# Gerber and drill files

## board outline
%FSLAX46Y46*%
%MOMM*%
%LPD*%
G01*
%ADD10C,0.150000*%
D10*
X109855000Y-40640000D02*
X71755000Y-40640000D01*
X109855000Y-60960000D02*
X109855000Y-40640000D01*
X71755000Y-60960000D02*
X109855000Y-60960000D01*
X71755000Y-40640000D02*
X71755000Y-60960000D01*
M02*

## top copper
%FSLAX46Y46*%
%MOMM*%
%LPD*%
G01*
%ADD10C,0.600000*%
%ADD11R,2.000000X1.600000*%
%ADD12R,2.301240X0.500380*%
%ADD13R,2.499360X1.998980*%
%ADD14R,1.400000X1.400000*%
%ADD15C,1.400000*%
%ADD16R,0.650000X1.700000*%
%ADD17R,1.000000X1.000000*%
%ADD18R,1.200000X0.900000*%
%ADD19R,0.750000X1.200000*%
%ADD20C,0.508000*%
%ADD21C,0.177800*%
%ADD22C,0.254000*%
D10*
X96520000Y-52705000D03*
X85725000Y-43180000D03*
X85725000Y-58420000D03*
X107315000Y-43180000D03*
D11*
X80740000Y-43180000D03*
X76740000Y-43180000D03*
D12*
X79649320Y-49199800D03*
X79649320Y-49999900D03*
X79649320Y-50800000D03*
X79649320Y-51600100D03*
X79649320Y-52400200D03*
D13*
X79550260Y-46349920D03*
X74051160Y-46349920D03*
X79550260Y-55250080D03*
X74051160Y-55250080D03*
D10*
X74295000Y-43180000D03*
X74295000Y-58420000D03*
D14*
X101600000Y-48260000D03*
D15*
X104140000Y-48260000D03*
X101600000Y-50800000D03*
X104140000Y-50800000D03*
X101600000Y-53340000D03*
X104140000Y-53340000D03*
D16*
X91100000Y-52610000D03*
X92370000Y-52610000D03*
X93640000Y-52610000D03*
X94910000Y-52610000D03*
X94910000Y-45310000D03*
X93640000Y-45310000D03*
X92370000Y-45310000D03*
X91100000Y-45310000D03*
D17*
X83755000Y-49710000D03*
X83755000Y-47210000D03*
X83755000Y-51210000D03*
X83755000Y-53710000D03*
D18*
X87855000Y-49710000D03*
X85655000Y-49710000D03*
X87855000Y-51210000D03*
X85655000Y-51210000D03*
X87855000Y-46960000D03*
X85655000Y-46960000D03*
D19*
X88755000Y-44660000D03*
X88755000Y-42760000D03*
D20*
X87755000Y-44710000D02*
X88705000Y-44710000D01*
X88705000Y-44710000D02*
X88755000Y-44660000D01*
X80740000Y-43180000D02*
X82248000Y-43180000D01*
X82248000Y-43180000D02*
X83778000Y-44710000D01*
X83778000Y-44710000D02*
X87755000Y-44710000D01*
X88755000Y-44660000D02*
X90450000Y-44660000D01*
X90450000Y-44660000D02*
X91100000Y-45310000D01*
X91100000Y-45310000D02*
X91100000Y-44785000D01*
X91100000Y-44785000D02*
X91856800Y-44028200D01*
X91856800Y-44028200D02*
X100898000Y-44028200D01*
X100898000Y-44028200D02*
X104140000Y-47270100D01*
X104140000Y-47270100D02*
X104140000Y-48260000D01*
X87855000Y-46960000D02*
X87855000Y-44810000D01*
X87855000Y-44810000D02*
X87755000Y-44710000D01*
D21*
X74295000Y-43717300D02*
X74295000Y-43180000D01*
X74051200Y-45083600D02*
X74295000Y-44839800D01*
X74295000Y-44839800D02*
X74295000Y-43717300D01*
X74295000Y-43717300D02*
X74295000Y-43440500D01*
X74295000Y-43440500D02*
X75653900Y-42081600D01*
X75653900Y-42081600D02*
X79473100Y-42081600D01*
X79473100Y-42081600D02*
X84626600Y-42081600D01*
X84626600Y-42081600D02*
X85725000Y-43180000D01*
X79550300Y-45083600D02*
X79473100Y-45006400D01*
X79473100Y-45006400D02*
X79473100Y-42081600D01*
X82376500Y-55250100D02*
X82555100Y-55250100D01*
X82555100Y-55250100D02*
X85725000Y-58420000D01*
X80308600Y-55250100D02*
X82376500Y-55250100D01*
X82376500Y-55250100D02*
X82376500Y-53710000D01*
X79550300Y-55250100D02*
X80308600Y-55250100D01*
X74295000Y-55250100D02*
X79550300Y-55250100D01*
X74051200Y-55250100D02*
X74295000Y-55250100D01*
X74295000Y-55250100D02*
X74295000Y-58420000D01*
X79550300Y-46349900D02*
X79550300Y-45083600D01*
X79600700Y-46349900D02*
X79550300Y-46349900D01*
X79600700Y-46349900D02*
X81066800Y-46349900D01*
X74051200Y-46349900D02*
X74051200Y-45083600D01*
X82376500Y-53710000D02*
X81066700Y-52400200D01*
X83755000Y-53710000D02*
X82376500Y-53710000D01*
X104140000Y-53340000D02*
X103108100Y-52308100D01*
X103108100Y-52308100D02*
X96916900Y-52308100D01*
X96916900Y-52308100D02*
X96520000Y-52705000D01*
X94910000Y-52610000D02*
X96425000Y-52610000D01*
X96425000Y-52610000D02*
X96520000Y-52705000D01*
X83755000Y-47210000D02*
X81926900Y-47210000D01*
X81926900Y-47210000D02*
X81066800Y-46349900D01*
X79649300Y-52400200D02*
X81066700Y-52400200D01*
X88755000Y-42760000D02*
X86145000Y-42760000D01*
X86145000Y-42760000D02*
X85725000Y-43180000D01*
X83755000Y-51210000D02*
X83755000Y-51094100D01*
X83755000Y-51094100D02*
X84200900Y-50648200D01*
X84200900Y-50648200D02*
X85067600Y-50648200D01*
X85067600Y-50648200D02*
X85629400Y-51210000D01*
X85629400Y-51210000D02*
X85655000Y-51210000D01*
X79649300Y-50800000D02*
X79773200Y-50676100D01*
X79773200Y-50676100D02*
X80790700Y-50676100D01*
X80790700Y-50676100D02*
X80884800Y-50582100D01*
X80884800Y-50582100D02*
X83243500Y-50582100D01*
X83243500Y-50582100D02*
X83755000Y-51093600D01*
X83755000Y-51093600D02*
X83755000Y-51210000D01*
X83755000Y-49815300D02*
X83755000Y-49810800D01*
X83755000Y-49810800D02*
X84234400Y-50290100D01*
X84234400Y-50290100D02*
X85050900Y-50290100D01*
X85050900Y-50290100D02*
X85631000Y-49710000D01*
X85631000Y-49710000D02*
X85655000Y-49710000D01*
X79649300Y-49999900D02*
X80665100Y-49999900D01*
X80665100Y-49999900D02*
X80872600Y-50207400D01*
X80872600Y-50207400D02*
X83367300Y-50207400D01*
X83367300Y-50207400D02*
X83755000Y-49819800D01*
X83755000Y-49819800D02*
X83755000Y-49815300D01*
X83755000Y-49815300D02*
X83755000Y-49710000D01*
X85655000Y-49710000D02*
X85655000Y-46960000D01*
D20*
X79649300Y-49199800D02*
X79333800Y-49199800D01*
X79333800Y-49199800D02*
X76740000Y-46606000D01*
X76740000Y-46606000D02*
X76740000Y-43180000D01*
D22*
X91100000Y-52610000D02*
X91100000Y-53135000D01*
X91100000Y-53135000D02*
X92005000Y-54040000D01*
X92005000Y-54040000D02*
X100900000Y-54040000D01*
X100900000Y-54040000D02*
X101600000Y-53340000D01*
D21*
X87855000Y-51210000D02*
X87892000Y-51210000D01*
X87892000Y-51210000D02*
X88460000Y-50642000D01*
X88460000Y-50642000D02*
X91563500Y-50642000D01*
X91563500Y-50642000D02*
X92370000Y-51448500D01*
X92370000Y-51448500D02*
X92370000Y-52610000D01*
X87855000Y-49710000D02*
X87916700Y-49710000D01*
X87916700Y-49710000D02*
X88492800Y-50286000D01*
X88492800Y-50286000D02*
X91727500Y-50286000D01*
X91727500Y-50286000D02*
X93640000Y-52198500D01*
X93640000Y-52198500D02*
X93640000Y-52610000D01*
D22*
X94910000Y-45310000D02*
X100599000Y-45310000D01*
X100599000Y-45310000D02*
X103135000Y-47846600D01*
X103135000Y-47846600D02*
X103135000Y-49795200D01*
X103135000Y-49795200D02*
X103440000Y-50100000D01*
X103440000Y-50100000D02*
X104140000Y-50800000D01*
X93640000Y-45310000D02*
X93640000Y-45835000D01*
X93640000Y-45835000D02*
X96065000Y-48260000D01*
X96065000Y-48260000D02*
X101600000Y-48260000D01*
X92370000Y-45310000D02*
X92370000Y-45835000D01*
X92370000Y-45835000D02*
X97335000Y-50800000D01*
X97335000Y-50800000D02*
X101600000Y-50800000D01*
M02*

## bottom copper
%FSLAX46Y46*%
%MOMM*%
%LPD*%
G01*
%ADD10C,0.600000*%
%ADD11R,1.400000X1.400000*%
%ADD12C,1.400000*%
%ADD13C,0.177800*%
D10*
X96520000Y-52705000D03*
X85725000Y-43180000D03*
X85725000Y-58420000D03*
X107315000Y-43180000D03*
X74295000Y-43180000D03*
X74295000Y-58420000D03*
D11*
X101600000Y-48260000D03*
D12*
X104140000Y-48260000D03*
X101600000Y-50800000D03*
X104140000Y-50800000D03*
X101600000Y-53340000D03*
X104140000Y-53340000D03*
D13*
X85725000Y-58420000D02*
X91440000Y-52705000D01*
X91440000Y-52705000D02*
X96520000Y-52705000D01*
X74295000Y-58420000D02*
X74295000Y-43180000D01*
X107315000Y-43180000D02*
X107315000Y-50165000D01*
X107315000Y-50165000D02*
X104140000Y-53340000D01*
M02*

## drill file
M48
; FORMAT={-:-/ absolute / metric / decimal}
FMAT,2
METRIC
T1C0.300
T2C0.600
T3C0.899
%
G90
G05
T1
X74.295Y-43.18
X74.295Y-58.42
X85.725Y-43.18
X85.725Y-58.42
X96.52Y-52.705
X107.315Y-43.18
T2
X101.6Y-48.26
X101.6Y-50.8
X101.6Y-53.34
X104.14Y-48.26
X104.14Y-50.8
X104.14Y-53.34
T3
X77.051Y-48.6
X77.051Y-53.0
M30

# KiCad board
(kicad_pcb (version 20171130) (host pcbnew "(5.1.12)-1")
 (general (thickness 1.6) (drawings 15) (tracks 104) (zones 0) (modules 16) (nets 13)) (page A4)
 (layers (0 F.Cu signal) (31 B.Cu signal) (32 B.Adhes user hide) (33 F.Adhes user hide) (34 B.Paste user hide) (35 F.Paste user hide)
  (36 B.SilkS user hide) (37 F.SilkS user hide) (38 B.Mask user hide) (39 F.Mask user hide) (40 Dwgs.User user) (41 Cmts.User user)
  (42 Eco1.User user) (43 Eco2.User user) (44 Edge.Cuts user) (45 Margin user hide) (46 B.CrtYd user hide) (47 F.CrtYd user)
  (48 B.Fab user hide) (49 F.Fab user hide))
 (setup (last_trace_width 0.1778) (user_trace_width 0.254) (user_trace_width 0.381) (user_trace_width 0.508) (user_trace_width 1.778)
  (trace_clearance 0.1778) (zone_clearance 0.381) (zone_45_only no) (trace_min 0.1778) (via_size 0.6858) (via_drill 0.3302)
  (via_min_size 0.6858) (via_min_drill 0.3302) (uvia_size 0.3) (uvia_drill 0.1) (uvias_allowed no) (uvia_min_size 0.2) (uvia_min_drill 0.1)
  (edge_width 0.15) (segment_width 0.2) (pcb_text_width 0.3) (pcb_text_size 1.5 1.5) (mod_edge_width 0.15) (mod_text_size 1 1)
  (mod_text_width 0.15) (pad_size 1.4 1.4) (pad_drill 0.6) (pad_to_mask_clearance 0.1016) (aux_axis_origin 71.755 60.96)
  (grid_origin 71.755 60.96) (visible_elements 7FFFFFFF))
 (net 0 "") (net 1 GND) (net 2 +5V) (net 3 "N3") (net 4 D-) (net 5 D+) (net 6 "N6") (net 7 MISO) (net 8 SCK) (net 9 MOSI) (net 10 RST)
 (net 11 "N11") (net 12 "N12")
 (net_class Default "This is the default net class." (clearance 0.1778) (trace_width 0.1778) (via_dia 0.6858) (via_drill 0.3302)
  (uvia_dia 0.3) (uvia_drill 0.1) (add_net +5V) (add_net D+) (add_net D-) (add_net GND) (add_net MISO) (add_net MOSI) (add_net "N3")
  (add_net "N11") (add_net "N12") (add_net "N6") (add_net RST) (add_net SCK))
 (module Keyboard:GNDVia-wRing (layer F.Cu) (at 96.52 52.705)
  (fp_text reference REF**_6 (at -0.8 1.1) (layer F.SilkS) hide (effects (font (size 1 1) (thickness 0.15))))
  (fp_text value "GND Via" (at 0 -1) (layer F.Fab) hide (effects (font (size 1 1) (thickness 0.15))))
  (pad GND thru_hole circle (at 0 0) (size 0.6 0.6) (drill 0.3) (layers *.Cu) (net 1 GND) (zone_connect 2)))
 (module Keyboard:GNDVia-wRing (layer F.Cu) (at 85.725 43.18)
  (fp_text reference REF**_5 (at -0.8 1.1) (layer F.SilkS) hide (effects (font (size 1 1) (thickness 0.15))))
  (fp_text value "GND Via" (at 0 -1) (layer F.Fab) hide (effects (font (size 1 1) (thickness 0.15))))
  (pad GND thru_hole circle (at 0 0) (size 0.6 0.6) (drill 0.3) (layers *.Cu) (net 1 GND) (zone_connect 2)))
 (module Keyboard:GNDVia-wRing (layer F.Cu) (at 85.725 58.42)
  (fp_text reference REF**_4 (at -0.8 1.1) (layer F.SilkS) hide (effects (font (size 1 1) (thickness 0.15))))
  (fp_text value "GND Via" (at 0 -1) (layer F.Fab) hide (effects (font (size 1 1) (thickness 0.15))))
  (pad GND thru_hole circle (at 0 0) (size 0.6 0.6) (drill 0.3) (layers *.Cu) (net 1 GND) (zone_connect 2)))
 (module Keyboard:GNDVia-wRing (layer F.Cu) (at 107.315 43.18)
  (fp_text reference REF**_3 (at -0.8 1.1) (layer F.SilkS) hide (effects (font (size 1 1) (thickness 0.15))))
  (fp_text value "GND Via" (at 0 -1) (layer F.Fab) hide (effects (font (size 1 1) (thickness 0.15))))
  (pad GND thru_hole circle (at 0 0) (size 0.6 0.6) (drill 0.3) (layers *.Cu) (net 1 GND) (zone_connect 2)))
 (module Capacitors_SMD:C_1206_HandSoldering (layer F.Cu) (at 78.74 43.18 180)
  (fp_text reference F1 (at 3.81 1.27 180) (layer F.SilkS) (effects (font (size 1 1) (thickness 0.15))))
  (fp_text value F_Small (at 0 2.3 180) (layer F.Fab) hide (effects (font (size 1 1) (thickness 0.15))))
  (pad 1 smd rect (at -2 0 180) (size 2 1.6) (layers F.Cu F.Paste F.Mask) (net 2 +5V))
  (pad 2 smd rect (at 2 0 180) (size 2 1.6) (layers F.Cu F.Paste F.Mask) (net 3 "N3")))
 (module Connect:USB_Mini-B (layer F.Cu) (at 76.2 50.8)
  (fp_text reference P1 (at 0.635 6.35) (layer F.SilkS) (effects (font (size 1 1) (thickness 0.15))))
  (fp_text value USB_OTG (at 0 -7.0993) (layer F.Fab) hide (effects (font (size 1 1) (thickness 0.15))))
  (pad 1 smd rect (at 3.44932 -1.6002) (size 2.30124 0.50038) (layers F.Cu F.Paste F.Mask) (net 3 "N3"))
  (pad 2 smd rect (at 3.44932 -0.8001) (size 2.30124 0.50038) (layers F.Cu F.Paste F.Mask) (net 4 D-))
  (pad 3 smd rect (at 3.44932 0) (size 2.30124 0.50038) (layers F.Cu F.Paste F.Mask) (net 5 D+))
  (pad 4 smd rect (at 3.44932 0.8001) (size 2.30124 0.50038) (layers F.Cu F.Paste F.Mask) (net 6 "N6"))
  (pad 5 smd rect (at 3.44932 1.6002) (size 2.30124 0.50038) (layers F.Cu F.Paste F.Mask) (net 1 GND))
  (pad 6 smd rect (at 3.35026 -4.45008) (size 2.49936 1.99898) (layers F.Cu F.Paste F.Mask) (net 1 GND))
  (pad 6 smd rect (at -2.14884 -4.45008) (size 2.49936 1.99898) (layers F.Cu F.Paste F.Mask) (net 1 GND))
  (pad 6 smd rect (at 3.35026 4.45008) (size 2.49936 1.99898) (layers F.Cu F.Paste F.Mask) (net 1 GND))
  (pad 6 smd rect (at -2.14884 4.45008) (size 2.49936 1.99898) (layers F.Cu F.Paste F.Mask) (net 1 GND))
  (pad "" np_thru_hole circle (at 0.8509 -2.19964) (size 0.89916 0.89916) (drill 0.89916) (layers *.Cu *.Mask F.SilkS))
  (pad "" np_thru_hole circle (at 0.8509 2.19964) (size 0.89916 0.89916) (drill 0.89916) (layers *.Cu *.Mask F.SilkS)))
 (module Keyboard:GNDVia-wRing (layer F.Cu) (at 74.295 43.18)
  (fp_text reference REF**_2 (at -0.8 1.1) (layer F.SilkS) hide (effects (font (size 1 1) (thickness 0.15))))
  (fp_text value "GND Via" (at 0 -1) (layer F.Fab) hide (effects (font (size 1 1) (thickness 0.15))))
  (pad GND thru_hole circle (at 0 0) (size 0.6 0.6) (drill 0.3) (layers *.Cu) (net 1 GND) (zone_connect 2)))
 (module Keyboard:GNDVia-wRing (layer F.Cu) (at 74.295 58.42)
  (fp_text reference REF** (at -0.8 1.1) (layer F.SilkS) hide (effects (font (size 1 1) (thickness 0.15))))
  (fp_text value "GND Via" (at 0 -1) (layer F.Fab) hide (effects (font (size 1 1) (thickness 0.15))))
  (pad GND thru_hole circle (at 0 0) (size 0.6 0.6) (drill 0.3) (layers *.Cu) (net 1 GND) (zone_connect 2)))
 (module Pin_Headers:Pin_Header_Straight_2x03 (layer F.Cu) (at 101.6 48.26)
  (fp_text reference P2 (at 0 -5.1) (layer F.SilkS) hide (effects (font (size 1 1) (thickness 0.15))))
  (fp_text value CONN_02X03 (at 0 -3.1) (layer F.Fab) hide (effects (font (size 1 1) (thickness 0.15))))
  (pad 1 thru_hole rect (at 0 0) (size 1.4 1.4) (drill 0.6) (layers *.Cu *.Mask F.SilkS) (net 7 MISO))
  (pad 2 thru_hole circle (at 2.54 0) (size 1.4 1.4) (drill 0.6) (layers *.Cu *.Mask F.SilkS) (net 2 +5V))
  (pad 3 thru_hole circle (at 0 2.54) (size 1.4 1.4) (drill 0.6) (layers *.Cu *.Mask F.SilkS) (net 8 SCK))
  (pad 4 thru_hole circle (at 2.54 2.54) (size 1.4 1.4) (drill 0.6) (layers *.Cu *.Mask F.SilkS) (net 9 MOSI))
  (pad 5 thru_hole circle (at 0 5.08) (size 1.4 1.4) (drill 0.6) (layers *.Cu *.Mask F.SilkS) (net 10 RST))
  (pad 6 thru_hole circle (at 2.54 5.08) (size 1.4 1.4) (drill 0.6) (layers *.Cu *.Mask F.SilkS) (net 1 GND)))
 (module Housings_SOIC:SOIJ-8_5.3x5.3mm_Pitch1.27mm (layer F.Cu) (at 93.005 48.96 90)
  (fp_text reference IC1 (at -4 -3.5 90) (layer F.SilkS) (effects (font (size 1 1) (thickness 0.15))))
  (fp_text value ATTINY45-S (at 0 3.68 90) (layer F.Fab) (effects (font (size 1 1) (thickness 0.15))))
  (pad 1 smd rect (at -3.65 -1.905 90) (size 1.7 0.65) (layers F.Cu F.Paste F.Mask) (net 10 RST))
  (pad 2 smd rect (at -3.65 -0.635 90) (size 1.7 0.65) (layers F.Cu F.Paste F.Mask) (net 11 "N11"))
  (pad 3 smd rect (at -3.65 0.635 90) (size 1.7 0.65) (layers F.Cu F.Paste F.Mask) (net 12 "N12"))
  (pad 4 smd rect (at -3.65 1.905 90) (size 1.7 0.65) (layers F.Cu F.Paste F.Mask) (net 1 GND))
  (pad 5 smd rect (at 3.65 1.905 90) (size 1.7 0.65) (layers F.Cu F.Paste F.Mask) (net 9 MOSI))
  (pad 6 smd rect (at 3.65 0.635 90) (size 1.7 0.65) (layers F.Cu F.Paste F.Mask) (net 7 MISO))
  (pad 7 smd rect (at 3.65 -0.635 90) (size 1.7 0.65) (layers F.Cu F.Paste F.Mask) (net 8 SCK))
  (pad 8 smd rect (at 3.65 -1.905 90) (size 1.7 0.65) (layers F.Cu F.Paste F.Mask) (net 2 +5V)))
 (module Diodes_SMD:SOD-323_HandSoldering (layer F.Cu) (at 83.755 48.46 90)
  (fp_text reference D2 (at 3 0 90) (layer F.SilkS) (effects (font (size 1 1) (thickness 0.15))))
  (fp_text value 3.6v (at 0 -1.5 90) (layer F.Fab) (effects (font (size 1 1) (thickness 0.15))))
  (pad 1 smd rect (at -1.25 0 90) (size 1 1) (layers F.Cu F.Paste F.Mask) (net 4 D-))
  (pad 2 smd rect (at 1.25 0 90) (size 1 1) (layers F.Cu F.Paste F.Mask) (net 1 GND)))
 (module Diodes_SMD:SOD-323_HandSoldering (layer F.Cu) (at 83.755 52.46 270)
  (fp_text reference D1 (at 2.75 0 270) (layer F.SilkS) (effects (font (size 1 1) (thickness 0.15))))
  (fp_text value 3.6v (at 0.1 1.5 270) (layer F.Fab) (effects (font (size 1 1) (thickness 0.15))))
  (pad 1 smd rect (at -1.25 0 270) (size 1 1) (layers F.Cu F.Paste F.Mask) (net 5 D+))
  (pad 2 smd rect (at 1.25 0 270) (size 1 1) (layers F.Cu F.Paste F.Mask) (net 1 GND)))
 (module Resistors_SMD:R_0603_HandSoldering (layer F.Cu) (at 86.755 49.71 180)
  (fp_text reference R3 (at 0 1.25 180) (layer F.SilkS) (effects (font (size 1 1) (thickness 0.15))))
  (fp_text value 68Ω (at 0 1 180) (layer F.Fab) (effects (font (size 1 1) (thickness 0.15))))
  (pad 1 smd rect (at -1.1 0 180) (size 1.2 0.9) (layers F.Cu F.Paste F.Mask) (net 12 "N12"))
  (pad 2 smd rect (at 1.1 0 180) (size 1.2 0.9) (layers F.Cu F.Paste F.Mask) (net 4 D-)))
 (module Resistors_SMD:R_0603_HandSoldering (layer F.Cu) (at 86.755 51.21 180)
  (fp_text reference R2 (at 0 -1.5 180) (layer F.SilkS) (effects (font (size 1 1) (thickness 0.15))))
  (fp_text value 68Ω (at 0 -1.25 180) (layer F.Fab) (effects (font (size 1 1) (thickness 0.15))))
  (pad 1 smd rect (at -1.1 0 180) (size 1.2 0.9) (layers F.Cu F.Paste F.Mask) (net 11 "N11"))
  (pad 2 smd rect (at 1.1 0 180) (size 1.2 0.9) (layers F.Cu F.Paste F.Mask) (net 5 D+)))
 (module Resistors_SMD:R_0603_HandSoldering (layer F.Cu) (at 86.755 46.96 180)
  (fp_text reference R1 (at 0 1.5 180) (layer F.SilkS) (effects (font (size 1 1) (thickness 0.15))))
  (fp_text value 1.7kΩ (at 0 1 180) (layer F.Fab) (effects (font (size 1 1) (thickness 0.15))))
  (pad 1 smd rect (at -1.1 0 180) (size 1.2 0.9) (layers F.Cu F.Paste F.Mask) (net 2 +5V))
  (pad 2 smd rect (at 1.1 0 180) (size 1.2 0.9) (layers F.Cu F.Paste F.Mask) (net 4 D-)))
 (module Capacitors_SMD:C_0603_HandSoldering (layer F.Cu) (at 88.755 43.71 90)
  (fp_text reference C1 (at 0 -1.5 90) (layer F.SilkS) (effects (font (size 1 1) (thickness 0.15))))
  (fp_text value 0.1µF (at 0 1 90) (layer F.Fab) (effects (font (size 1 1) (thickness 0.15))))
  (pad 1 smd rect (at -0.95 0 90) (size 1.2 0.75) (layers F.Cu F.Paste F.Mask) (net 2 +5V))
  (pad 2 smd rect (at 0.95 0 90) (size 1.2 0.75) (layers F.Cu F.Paste F.Mask) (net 1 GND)))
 (gr_line (start 109.855 40.64) (end 71.755 40.64) (layer Edge.Cuts) (width 0.15))
 (gr_line (start 109.855 60.96) (end 109.855 40.64) (layer Edge.Cuts) (width 0.15))
 (gr_line (start 71.755 60.96) (end 109.855 60.96) (layer Edge.Cuts) (width 0.15))
 (gr_line (start 71.755 40.64) (end 71.755 60.96) (layer Edge.Cuts) (width 0.15))
 (segment (start 87.755 44.71) (end 88.705 44.71) (width 0.508) (layer F.Cu) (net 2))
 (segment (start 88.705 44.71) (end 88.755 44.66) (width 0.508) (layer F.Cu) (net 2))
 (segment (start 80.74 43.18) (end 82.248 43.18) (width 0.508) (layer F.Cu) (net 2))
 (segment (start 82.248 43.18) (end 83.778 44.71) (width 0.508) (layer F.Cu) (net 2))
 (segment (start 83.778 44.71) (end 87.755 44.71) (width 0.508) (layer F.Cu) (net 2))
 (segment (start 88.755 44.66) (end 90.45 44.66) (width 0.508) (layer F.Cu) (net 2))
 (segment (start 90.45 44.66) (end 91.1 45.31) (width 0.508) (layer F.Cu) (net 2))
 (segment (start 91.1 45.31) (end 91.1 44.785) (width 0.508) (layer F.Cu) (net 2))
 (segment (start 91.1 44.785) (end 91.8568 44.0282) (width 0.508) (layer F.Cu) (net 2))
 (segment (start 91.8568 44.0282) (end 100.898 44.0282) (width 0.508) (layer F.Cu) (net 2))
 (segment (start 100.898 44.0282) (end 104.14 47.2701) (width 0.508) (layer F.Cu) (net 2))
 (segment (start 104.14 47.2701) (end 104.14 48.26) (width 0.508) (layer F.Cu) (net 2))
 (segment (start 87.855 46.96) (end 87.855 44.81) (width 0.508) (layer F.Cu) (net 2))
 (segment (start 87.855 44.81) (end 87.755 44.71) (width 0.508) (layer F.Cu) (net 2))
 (segment (start 85.725 58.42) (end 91.44 52.705) (width 0.1778) (layer B.Cu) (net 1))
 (segment (start 91.44 52.705) (end 96.52 52.705) (width 0.1778) (layer B.Cu) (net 1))
 (segment (start 74.295 58.42) (end 74.295 43.18) (width 0.1778) (layer B.Cu) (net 1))
 (segment (start 107.315 43.18) (end 107.315 50.165) (width 0.1778) (layer B.Cu) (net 1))
 (segment (start 107.315 50.165) (end 104.14 53.34) (width 0.1778) (layer B.Cu) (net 1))
 (segment (start 74.295 43.7173) (end 74.295 43.18) (width 0.1778) (layer F.Cu) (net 1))
 (segment (start 74.0512 45.0836) (end 74.295 44.8398) (width 0.1778) (layer F.Cu) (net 1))
 (segment (start 74.295 44.8398) (end 74.295 43.7173) (width 0.1778) (layer F.Cu) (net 1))
 (segment (start 74.295 43.7173) (end 74.295 43.4405) (width 0.1778) (layer F.Cu) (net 1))
 (segment (start 74.295 43.4405) (end 75.6539 42.0816) (width 0.1778) (layer F.Cu) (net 1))
 (segment (start 75.6539 42.0816) (end 79.4731 42.0816) (width 0.1778) (layer F.Cu) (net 1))
 (segment (start 79.4731 42.0816) (end 84.6266 42.0816) (width 0.1778) (layer F.Cu) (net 1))
 (segment (start 84.6266 42.0816) (end 85.725 43.18) (width 0.1778) (layer F.Cu) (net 1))
 (segment (start 79.5503 45.0836) (end 79.4731 45.0064) (width 0.1778) (layer F.Cu) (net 1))
 (segment (start 79.4731 45.0064) (end 79.4731 42.0816) (width 0.1778) (layer F.Cu) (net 1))
 (segment (start 82.3765 55.2501) (end 82.5551 55.2501) (width 0.1778) (layer F.Cu) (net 1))
 (segment (start 82.5551 55.2501) (end 85.725 58.42) (width 0.1778) (layer F.Cu) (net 1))
 (segment (start 80.3086 55.2501) (end 82.3765 55.2501) (width 0.1778) (layer F.Cu) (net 1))
 (segment (start 82.3765 55.2501) (end 82.3765 53.71) (width 0.1778) (layer F.Cu) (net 1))
 (segment (start 79.5503 55.2501) (end 80.3086 55.2501) (width 0.1778) (layer F.Cu) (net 1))
 (segment (start 74.295 55.2501) (end 79.5503 55.2501) (width 0.1778) (layer F.Cu) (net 1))
 (segment (start 74.0512 55.2501) (end 74.295 55.2501) (width 0.1778) (layer F.Cu) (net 1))
 (segment (start 74.295 55.2501) (end 74.295 58.42) (width 0.1778) (layer F.Cu) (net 1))
 (segment (start 79.5503 46.3499) (end 79.5503 45.0836) (width 0.1778) (layer F.Cu) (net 1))
 (segment (start 79.6007 46.3499) (end 79.5503 46.3499) (width 0.1778) (layer F.Cu) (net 1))
 (segment (start 79.6007 46.3499) (end 81.0668 46.3499) (width 0.1778) (layer F.Cu) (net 1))
 (segment (start 74.0512 46.3499) (end 74.0512 45.0836) (width 0.1778) (layer F.Cu) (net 1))
 (segment (start 82.3765 53.71) (end 81.0667 52.4002) (width 0.1778) (layer F.Cu) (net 1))
 (segment (start 83.755 53.71) (end 82.3765 53.71) (width 0.1778) (layer F.Cu) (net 1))
 (segment (start 104.14 53.34) (end 103.1081 52.3081) (width 0.1778) (layer F.Cu) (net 1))
 (segment (start 103.1081 52.3081) (end 96.9169 52.3081) (width 0.1778) (layer F.Cu) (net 1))
 (segment (start 96.9169 52.3081) (end 96.52 52.705) (width 0.1778) (layer F.Cu) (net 1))
 (segment (start 94.91 52.61) (end 96.425 52.61) (width 0.1778) (layer F.Cu) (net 1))
 (segment (start 96.425 52.61) (end 96.52 52.705) (width 0.1778) (layer F.Cu) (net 1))
 (segment (start 83.755 47.21) (end 81.9269 47.21) (width 0.1778) (layer F.Cu) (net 1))
 (segment (start 81.9269 47.21) (end 81.0668 46.3499) (width 0.1778) (layer F.Cu) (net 1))
 (segment (start 79.6493 52.4002) (end 81.0667 52.4002) (width 0.1778) (layer F.Cu) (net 1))
 (segment (start 88.755 42.76) (end 86.145 42.76) (width 0.1778) (layer F.Cu) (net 1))
 (segment (start 86.145 42.76) (end 85.725 43.18) (width 0.1778) (layer F.Cu) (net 1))
 (segment (start 83.755 51.21) (end 83.755 51.0941) (width 0.1778) (layer F.Cu) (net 5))
 (segment (start 83.755 51.0941) (end 84.2009 50.6482) (width 0.1778) (layer F.Cu) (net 5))
 (segment (start 84.2009 50.6482) (end 85.0676 50.6482) (width 0.1778) (layer F.Cu) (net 5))
 (segment (start 85.0676 50.6482) (end 85.6294 51.21) (width 0.1778) (layer F.Cu) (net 5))
 (segment (start 85.6294 51.21) (end 85.655 51.21) (width 0.1778) (layer F.Cu) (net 5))
 (segment (start 79.6493 50.8) (end 79.7732 50.6761) (width 0.1778) (layer F.Cu) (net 5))
 (segment (start 79.7732 50.6761) (end 80.7907 50.6761) (width 0.1778) (layer F.Cu) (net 5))
 (segment (start 80.7907 50.6761) (end 80.8848 50.5821) (width 0.1778) (layer F.Cu) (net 5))
 (segment (start 80.8848 50.5821) (end 83.2435 50.5821) (width 0.1778) (layer F.Cu) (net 5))
 (segment (start 83.2435 50.5821) (end 83.755 51.0936) (width 0.1778) (layer F.Cu) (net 5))
 (segment (start 83.755 51.0936) (end 83.755 51.21) (width 0.1778) (layer F.Cu) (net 5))
 (segment (start 83.755 49.8153) (end 83.755 49.8108) (width 0.1778) (layer F.Cu) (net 4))
 (segment (start 83.755 49.8108) (end 84.2344 50.2901) (width 0.1778) (layer F.Cu) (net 4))
 (segment (start 84.2344 50.2901) (end 85.0509 50.2901) (width 0.1778) (layer F.Cu) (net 4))
 (segment (start 85.0509 50.2901) (end 85.631 49.71) (width 0.1778) (layer F.Cu) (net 4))
 (segment (start 85.631 49.71) (end 85.655 49.71) (width 0.1778) (layer F.Cu) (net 4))
 (segment (start 79.6493 49.9999) (end 80.6651 49.9999) (width 0.1778) (layer F.Cu) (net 4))
 (segment (start 80.6651 49.9999) (end 80.8726 50.2074) (width 0.1778) (layer F.Cu) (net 4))
 (segment (start 80.8726 50.2074) (end 83.3673 50.2074) (width 0.1778) (layer F.Cu) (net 4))
 (segment (start 83.3673 50.2074) (end 83.755 49.8198) (width 0.1778) (layer F.Cu) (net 4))
 (segment (start 83.755 49.8198) (end 83.755 49.8153) (width 0.1778) (layer F.Cu) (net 4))
 (segment (start 83.755 49.8153) (end 83.755 49.71) (width 0.1778) (layer F.Cu) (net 4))
 (segment (start 85.655 49.71) (end 85.655 46.96) (width 0.1778) (layer F.Cu) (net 4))
 (segment (start 79.6493 49.1998) (end 79.3338 49.1998) (width 0.508) (layer F.Cu) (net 3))
 (segment (start 79.3338 49.1998) (end 76.74 46.606) (width 0.508) (layer F.Cu) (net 3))
 (segment (start 76.74 46.606) (end 76.74 43.18) (width 0.508) (layer F.Cu) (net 3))
 (segment (start 91.1 52.61) (end 91.1 53.135) (width 0.254) (layer F.Cu) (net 10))
 (segment (start 91.1 53.135) (end 92.005 54.04) (width 0.254) (layer F.Cu) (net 10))
 (segment (start 92.005 54.04) (end 100.9 54.04) (width 0.254) (layer F.Cu) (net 10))
 (segment (start 100.9 54.04) (end 101.6 53.34) (width 0.254) (layer F.Cu) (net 10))
 (segment (start 87.855 51.21) (end 87.892 51.21) (width 0.1778) (layer F.Cu) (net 11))
 (segment (start 87.892 51.21) (end 88.46 50.642) (width 0.1778) (layer F.Cu) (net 11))
 (segment (start 88.46 50.642) (end 91.5635 50.642) (width 0.1778) (layer F.Cu) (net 11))
 (segment (start 91.5635 50.642) (end 92.37 51.4485) (width 0.1778) (layer F.Cu) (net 11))
 (segment (start 92.37 51.4485) (end 92.37 52.61) (width 0.1778) (layer F.Cu) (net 11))
 (segment (start 87.855 49.71) (end 87.9167 49.71) (width 0.1778) (layer F.Cu) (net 12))
 (segment (start 87.9167 49.71) (end 88.4928 50.286) (width 0.1778) (layer F.Cu) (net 12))
 (segment (start 88.4928 50.286) (end 91.7275 50.286) (width 0.1778) (layer F.Cu) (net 12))
 (segment (start 91.7275 50.286) (end 93.64 52.1985) (width 0.1778) (layer F.Cu) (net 12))
 (segment (start 93.64 52.1985) (end 93.64 52.61) (width 0.1778) (layer F.Cu) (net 12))
 (segment (start 94.91 45.31) (end 100.599 45.31) (width 0.254) (layer F.Cu) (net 9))
 (segment (start 100.599 45.31) (end 103.135 47.8466) (width 0.254) (layer F.Cu) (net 9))
 (segment (start 103.135 47.8466) (end 103.135 49.7952) (width 0.254) (layer F.Cu) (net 9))
 (segment (start 103.135 49.7952) (end 103.44 50.1) (width 0.254) (layer F.Cu) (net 9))
 (segment (start 103.44 50.1) (end 104.14 50.8) (width 0.254) (layer F.Cu) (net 9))
 (segment (start 93.64 45.31) (end 93.64 45.835) (width 0.254) (layer F.Cu) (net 7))
 (segment (start 93.64 45.835) (end 96.065 48.26) (width 0.254) (layer F.Cu) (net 7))
 (segment (start 96.065 48.26) (end 101.6 48.26) (width 0.254) (layer F.Cu) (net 7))
 (segment (start 92.37 45.31) (end 92.37 45.835) (width 0.254) (layer F.Cu) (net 8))
 (segment (start 92.37 45.835) (end 97.335 50.8) (width 0.254) (layer F.Cu) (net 8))
 (segment (start 97.335 50.8) (end 101.6 50.8) (width 0.254) (layer F.Cu) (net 8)))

